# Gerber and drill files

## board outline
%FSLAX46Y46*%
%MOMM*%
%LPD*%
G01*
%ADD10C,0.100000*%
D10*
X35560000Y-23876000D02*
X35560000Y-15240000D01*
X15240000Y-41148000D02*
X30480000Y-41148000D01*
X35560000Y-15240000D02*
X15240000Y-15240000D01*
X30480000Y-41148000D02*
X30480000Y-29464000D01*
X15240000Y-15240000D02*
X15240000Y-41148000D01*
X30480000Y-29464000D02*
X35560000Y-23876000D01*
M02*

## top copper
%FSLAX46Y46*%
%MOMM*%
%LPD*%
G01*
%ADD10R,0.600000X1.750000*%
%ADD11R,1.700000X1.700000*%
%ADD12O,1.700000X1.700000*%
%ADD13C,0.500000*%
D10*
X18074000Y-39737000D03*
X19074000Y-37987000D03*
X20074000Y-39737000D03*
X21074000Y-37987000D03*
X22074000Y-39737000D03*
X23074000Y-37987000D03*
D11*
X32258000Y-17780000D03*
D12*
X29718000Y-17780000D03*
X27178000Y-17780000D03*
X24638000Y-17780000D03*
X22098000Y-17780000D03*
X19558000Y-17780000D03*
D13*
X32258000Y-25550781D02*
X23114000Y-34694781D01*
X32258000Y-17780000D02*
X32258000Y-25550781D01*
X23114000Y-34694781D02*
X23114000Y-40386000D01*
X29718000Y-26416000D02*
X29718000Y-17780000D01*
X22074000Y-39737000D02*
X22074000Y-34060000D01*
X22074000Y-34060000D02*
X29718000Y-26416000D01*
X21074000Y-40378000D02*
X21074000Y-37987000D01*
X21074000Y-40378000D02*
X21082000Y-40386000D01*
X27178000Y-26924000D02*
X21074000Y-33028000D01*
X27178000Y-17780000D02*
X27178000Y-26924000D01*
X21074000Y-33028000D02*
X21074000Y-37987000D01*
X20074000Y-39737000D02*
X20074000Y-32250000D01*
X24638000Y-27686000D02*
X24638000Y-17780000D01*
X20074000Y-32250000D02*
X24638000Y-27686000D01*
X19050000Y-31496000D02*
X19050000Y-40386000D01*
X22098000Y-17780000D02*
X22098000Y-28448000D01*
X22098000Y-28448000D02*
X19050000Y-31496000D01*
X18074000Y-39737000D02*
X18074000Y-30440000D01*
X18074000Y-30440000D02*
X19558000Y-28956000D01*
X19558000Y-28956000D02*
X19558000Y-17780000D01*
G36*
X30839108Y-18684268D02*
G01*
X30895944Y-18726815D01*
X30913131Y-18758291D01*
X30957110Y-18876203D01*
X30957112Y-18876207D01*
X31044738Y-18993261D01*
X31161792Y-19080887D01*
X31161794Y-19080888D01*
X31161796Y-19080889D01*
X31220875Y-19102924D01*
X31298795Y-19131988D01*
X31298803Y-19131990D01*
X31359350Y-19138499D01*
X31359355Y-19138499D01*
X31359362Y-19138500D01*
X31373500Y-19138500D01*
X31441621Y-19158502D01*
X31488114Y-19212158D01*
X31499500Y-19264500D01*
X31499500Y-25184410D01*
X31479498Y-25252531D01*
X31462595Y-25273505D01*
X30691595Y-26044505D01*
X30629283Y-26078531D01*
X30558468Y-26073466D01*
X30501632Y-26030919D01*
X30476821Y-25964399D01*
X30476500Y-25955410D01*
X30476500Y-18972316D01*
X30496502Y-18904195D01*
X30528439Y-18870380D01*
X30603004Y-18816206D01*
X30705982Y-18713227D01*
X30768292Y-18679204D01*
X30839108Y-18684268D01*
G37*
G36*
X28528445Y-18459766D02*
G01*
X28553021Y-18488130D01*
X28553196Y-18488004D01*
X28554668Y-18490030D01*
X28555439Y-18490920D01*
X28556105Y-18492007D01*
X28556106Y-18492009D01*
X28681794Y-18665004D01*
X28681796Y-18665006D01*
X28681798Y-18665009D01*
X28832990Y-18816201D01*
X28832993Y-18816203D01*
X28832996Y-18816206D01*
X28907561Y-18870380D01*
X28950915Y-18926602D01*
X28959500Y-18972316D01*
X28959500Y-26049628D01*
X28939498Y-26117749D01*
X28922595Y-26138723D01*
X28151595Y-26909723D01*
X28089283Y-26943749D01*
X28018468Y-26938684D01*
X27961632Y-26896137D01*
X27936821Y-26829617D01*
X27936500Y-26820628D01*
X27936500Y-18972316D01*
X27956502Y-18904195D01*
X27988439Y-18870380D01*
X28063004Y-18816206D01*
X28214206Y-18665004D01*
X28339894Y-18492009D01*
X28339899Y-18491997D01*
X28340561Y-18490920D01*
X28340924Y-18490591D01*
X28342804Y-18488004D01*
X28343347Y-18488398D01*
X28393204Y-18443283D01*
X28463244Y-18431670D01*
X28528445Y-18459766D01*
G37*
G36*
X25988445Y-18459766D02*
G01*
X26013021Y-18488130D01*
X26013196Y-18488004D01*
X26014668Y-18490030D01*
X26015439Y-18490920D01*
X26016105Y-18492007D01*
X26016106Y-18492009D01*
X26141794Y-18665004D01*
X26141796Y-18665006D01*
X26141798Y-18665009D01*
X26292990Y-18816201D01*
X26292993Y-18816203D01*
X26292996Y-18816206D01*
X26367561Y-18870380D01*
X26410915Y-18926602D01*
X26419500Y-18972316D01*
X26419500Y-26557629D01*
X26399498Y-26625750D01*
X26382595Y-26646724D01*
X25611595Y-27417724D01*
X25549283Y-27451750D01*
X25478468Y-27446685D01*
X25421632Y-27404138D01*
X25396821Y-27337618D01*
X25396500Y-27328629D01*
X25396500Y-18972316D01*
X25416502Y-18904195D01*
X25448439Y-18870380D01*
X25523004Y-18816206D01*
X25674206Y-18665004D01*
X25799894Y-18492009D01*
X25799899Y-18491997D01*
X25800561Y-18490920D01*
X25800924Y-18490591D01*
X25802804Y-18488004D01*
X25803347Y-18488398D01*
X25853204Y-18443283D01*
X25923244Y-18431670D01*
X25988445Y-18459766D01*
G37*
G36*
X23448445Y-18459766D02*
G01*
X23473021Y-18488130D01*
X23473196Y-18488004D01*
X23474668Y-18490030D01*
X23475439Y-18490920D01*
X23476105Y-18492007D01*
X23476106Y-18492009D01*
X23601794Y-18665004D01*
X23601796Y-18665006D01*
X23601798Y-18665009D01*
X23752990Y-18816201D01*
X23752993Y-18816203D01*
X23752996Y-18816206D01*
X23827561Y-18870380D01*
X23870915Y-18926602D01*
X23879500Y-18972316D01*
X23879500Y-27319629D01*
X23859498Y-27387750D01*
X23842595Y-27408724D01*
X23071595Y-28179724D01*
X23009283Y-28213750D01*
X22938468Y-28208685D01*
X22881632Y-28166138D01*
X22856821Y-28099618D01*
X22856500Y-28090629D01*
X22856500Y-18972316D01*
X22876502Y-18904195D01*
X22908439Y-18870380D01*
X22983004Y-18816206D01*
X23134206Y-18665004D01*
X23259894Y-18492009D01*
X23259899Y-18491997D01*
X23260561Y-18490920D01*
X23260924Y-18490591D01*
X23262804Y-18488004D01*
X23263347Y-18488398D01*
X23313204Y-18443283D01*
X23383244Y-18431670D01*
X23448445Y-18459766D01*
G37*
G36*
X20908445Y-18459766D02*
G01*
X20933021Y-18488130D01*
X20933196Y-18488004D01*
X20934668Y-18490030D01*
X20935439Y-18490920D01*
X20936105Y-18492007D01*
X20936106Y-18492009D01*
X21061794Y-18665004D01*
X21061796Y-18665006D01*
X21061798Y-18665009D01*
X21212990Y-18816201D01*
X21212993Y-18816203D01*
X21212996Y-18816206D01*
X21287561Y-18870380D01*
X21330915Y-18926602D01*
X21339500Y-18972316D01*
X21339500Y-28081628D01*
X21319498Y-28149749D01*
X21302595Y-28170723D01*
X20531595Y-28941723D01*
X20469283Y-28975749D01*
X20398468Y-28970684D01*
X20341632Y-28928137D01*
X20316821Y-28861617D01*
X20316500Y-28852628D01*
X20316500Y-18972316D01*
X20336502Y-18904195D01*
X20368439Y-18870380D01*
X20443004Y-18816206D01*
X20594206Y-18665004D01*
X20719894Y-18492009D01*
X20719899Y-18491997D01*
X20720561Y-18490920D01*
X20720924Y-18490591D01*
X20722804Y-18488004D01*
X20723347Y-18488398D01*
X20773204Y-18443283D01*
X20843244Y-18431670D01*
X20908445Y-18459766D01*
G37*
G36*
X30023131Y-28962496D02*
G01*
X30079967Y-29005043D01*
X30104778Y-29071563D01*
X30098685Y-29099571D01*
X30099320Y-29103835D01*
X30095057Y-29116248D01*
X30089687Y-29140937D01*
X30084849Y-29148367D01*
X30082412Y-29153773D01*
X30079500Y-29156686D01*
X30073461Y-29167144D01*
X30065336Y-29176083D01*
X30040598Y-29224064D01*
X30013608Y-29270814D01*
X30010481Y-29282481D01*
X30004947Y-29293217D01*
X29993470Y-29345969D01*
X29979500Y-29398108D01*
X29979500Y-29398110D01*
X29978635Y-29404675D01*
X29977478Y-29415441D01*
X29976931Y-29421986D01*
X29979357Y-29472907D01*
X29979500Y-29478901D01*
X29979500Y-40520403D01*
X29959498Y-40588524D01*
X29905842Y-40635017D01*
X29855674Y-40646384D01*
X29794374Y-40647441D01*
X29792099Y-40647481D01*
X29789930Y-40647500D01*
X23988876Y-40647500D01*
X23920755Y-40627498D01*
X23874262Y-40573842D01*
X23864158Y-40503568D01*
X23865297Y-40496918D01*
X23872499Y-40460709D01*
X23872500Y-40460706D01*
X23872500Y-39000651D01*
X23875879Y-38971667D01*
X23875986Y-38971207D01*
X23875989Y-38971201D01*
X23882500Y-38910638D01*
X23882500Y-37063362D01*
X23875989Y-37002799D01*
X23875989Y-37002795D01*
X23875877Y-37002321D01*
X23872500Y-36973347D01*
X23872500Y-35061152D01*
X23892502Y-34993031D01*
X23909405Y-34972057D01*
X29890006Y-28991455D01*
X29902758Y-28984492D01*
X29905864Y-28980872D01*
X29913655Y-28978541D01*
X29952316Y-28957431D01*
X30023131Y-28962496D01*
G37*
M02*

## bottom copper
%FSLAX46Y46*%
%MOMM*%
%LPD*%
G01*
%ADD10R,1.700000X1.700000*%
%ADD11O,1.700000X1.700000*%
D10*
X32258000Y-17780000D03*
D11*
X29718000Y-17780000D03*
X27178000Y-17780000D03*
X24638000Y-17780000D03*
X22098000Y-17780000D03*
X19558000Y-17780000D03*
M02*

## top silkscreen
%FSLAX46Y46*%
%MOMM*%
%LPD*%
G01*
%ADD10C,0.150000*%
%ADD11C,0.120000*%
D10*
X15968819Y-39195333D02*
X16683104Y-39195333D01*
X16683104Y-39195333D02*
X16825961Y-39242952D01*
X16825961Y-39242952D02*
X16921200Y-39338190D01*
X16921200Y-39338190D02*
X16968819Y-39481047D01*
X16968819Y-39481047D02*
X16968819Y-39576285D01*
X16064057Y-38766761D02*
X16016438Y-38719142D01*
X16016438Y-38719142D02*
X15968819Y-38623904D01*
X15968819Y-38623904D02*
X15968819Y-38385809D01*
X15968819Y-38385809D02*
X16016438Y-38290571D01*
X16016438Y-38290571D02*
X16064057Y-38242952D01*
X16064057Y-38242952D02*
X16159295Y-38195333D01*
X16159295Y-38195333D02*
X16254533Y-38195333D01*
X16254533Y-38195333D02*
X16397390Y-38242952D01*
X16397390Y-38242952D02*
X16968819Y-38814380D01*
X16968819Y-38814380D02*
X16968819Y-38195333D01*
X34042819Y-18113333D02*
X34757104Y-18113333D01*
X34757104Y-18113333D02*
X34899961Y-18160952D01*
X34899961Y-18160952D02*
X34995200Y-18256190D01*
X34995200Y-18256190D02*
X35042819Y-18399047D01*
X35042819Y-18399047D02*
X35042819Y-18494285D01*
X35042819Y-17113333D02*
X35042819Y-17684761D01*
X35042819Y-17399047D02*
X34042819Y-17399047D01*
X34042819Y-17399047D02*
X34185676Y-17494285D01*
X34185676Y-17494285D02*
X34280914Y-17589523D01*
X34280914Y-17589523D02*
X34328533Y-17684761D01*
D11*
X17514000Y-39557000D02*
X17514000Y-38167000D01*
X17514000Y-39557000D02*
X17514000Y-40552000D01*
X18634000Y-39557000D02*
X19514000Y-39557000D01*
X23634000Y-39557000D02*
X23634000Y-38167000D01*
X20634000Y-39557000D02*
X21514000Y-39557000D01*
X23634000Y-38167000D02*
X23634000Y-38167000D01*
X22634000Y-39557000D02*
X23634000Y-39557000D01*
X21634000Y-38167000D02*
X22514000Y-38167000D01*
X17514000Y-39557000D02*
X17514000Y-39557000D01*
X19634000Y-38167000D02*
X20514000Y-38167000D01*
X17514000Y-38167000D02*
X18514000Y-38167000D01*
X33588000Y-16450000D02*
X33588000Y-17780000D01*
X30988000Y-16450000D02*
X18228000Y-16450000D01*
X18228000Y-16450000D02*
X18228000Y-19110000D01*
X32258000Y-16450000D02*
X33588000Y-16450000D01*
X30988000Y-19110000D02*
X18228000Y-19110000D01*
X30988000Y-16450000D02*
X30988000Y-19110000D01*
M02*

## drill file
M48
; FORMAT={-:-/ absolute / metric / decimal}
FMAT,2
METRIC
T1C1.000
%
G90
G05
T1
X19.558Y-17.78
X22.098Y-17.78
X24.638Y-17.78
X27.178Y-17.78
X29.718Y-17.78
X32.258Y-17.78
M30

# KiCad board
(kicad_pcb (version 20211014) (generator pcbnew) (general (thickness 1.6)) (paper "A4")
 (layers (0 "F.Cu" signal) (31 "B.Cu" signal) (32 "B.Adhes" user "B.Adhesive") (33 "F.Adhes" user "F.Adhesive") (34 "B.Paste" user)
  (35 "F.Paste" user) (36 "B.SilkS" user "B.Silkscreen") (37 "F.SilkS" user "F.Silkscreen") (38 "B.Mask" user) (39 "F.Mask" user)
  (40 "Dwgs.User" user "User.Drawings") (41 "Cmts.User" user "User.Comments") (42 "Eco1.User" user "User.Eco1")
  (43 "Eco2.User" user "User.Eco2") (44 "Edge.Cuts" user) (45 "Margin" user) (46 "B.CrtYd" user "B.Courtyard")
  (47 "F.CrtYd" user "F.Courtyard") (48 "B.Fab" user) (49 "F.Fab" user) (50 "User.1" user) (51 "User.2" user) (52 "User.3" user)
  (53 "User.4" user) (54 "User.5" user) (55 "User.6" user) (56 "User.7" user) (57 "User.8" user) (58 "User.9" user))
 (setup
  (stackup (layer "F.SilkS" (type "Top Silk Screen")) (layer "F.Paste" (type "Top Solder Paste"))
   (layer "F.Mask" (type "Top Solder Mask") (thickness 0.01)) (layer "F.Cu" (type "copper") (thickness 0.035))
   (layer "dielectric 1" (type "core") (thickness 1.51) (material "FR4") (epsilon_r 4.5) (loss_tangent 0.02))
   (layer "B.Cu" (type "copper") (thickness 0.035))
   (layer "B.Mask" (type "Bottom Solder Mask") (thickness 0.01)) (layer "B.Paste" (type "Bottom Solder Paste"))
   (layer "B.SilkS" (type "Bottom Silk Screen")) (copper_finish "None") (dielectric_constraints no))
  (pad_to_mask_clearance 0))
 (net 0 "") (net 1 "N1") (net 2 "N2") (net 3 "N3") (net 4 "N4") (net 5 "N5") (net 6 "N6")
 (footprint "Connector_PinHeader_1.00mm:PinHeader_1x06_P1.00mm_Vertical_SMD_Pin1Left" (layer "F.Cu") (at 20.574 38.862 90)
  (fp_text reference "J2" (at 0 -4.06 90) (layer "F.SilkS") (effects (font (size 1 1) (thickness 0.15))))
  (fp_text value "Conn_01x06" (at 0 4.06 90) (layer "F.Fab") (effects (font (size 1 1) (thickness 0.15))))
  (fp_line (start -0.695 -3.06) (end 0.695 -3.06) (layer "F.SilkS") (width 0.12))
  (fp_line (start -0.695 -3.06) (end -1.69 -3.06) (layer "F.SilkS") (width 0.12))
  (fp_line (start -0.695 -1.94) (end -0.695 -1.06) (layer "F.SilkS") (width 0.12))
  (fp_line (start -0.695 3.06) (end 0.695 3.06) (layer "F.SilkS") (width 0.12))
  (fp_line (start -0.695 0.06) (end -0.695 0.94) (layer "F.SilkS") (width 0.12))
  (fp_line (start 0.695 3.06) (end 0.695 3.06) (layer "F.SilkS") (width 0.12))
  (fp_line (start -0.695 2.06) (end -0.695 3.06) (layer "F.SilkS") (width 0.12))
  (fp_line (start 0.695 1.06) (end 0.695 1.94) (layer "F.SilkS") (width 0.12))
  (fp_line (start -0.695 -3.06) (end -0.695 -3.06) (layer "F.SilkS") (width 0.12))
  (fp_line (start 0.695 -0.94) (end 0.695 -0.06) (layer "F.SilkS") (width 0.12))
  (fp_line (start 0.695 -3.06) (end 0.695 -2.06) (layer "F.SilkS") (width 0.12))
  (pad "1" smd rect (at -0.875 -2.5 90) (size 1.75 0.6) (layers "F.Cu" "F.Paste" "F.Mask") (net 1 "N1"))
  (pad "2" smd rect (at 0.875 -1.5 90) (size 1.75 0.6) (layers "F.Cu" "F.Paste" "F.Mask") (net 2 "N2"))
  (pad "3" smd rect (at -0.875 -0.5 90) (size 1.75 0.6) (layers "F.Cu" "F.Paste" "F.Mask") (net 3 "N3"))
  (pad "4" smd rect (at 0.875 0.5 90) (size 1.75 0.6) (layers "F.Cu" "F.Paste" "F.Mask") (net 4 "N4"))
  (pad "5" smd rect (at -0.875 1.5 90) (size 1.75 0.6) (layers "F.Cu" "F.Paste" "F.Mask") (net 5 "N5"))
  (pad "6" smd rect (at 0.875 2.5 90) (size 1.75 0.6) (layers "F.Cu" "F.Paste" "F.Mask") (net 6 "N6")))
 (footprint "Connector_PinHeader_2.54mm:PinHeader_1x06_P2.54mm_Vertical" (layer "F.Cu") (at 32.258 17.78 -90)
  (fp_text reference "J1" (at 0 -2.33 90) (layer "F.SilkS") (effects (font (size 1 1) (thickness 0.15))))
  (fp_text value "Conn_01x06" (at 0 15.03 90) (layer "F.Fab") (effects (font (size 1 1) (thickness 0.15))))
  (fp_line (start -1.33 -1.33) (end 0 -1.33) (layer "F.SilkS") (width 0.12))
  (fp_line (start -1.33 1.27) (end -1.33 14.03) (layer "F.SilkS") (width 0.12))
  (fp_line (start -1.33 14.03) (end 1.33 14.03) (layer "F.SilkS") (width 0.12))
  (fp_line (start -1.33 0) (end -1.33 -1.33) (layer "F.SilkS") (width 0.12))
  (fp_line (start 1.33 1.27) (end 1.33 14.03) (layer "F.SilkS") (width 0.12))
  (fp_line (start -1.33 1.27) (end 1.33 1.27) (layer "F.SilkS") (width 0.12))
  (pad "1" thru_hole rect (at 0 0 270) (size 1.7 1.7) (drill 1) (layers *.Cu *.Mask) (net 6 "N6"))
  (pad "2" thru_hole oval (at 0 2.54 270) (size 1.7 1.7) (drill 1) (layers *.Cu *.Mask) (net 5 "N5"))
  (pad "3" thru_hole oval (at 0 5.08 270) (size 1.7 1.7) (drill 1) (layers *.Cu *.Mask) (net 4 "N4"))
  (pad "4" thru_hole oval (at 0 7.62 270) (size 1.7 1.7) (drill 1) (layers *.Cu *.Mask) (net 3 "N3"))
  (pad "5" thru_hole oval (at 0 10.16 270) (size 1.7 1.7) (drill 1) (layers *.Cu *.Mask) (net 2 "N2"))
  (pad "6" thru_hole oval (at 0 12.7 270) (size 1.7 1.7) (drill 1) (layers *.Cu *.Mask) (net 1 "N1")))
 (gr_line (start 35.56 23.876) (end 35.56 15.24) (layer "Edge.Cuts") (width 0.1))
 (gr_line (start 15.24 41.148) (end 30.48 41.148) (layer "Edge.Cuts") (width 0.1))
 (gr_line (start 35.56 15.24) (end 15.24 15.24) (layer "Edge.Cuts") (width 0.1))
 (gr_line (start 30.48 41.148) (end 30.48 29.464) (layer "Edge.Cuts") (width 0.1))
 (gr_line (start 15.24 15.24) (end 15.24 41.148) (layer "Edge.Cuts") (width 0.1))
 (gr_line (start 30.48 29.464) (end 35.56 23.876) (layer "Edge.Cuts") (width 0.1))
 (segment (start 32.258 25.550781) (end 23.114 34.694781) (width 0.5) (layer "F.Cu") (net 6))
 (segment (start 32.258 17.78) (end 32.258 25.550781) (width 0.5) (layer "F.Cu") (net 6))
 (segment (start 23.114 34.694781) (end 23.114 40.386) (width 0.5) (layer "F.Cu") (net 6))
 (segment (start 29.718 26.416) (end 29.718 17.78) (width 0.5) (layer "F.Cu") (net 5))
 (segment (start 22.074 39.737) (end 22.074 34.06) (width 0.5) (layer "F.Cu") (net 5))
 (segment (start 22.074 34.06) (end 29.718 26.416) (width 0.5) (layer "F.Cu") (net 5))
 (segment (start 21.074 40.378) (end 21.074 37.987) (width 0.5) (layer "F.Cu") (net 4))
 (segment (start 21.074 40.378) (end 21.082 40.386) (width 0.5) (layer "F.Cu") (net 4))
 (segment (start 27.178 26.924) (end 21.074 33.028) (width 0.5) (layer "F.Cu") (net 4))
 (segment (start 27.178 17.78) (end 27.178 26.924) (width 0.5) (layer "F.Cu") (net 4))
 (segment (start 21.074 33.028) (end 21.074 37.987) (width 0.5) (layer "F.Cu") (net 4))
 (segment (start 20.074 39.737) (end 20.074 32.25) (width 0.5) (layer "F.Cu") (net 3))
 (segment (start 24.638 27.686) (end 24.638 17.78) (width 0.5) (layer "F.Cu") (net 3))
 (segment (start 20.074 32.25) (end 24.638 27.686) (width 0.5) (layer "F.Cu") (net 3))
 (segment (start 19.05 31.496) (end 19.05 40.386) (width 0.5) (layer "F.Cu") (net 2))
 (segment (start 22.098 17.78) (end 22.098 28.448) (width 0.5) (layer "F.Cu") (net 2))
 (segment (start 22.098 28.448) (end 19.05 31.496) (width 0.5) (layer "F.Cu") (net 2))
 (segment (start 18.074 39.737) (end 18.074 30.44) (width 0.5) (layer "F.Cu") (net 1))
 (segment (start 18.074 30.44) (end 19.558 28.956) (width 0.5) (layer "F.Cu") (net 1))
 (segment (start 19.558 28.956) (end 19.558 17.78) (width 0.5) (layer "F.Cu") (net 1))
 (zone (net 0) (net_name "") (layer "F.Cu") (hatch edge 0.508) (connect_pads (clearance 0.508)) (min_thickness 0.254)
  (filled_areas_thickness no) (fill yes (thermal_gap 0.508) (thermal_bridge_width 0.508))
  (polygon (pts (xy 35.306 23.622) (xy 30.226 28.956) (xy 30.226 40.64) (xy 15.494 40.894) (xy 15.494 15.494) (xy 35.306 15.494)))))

